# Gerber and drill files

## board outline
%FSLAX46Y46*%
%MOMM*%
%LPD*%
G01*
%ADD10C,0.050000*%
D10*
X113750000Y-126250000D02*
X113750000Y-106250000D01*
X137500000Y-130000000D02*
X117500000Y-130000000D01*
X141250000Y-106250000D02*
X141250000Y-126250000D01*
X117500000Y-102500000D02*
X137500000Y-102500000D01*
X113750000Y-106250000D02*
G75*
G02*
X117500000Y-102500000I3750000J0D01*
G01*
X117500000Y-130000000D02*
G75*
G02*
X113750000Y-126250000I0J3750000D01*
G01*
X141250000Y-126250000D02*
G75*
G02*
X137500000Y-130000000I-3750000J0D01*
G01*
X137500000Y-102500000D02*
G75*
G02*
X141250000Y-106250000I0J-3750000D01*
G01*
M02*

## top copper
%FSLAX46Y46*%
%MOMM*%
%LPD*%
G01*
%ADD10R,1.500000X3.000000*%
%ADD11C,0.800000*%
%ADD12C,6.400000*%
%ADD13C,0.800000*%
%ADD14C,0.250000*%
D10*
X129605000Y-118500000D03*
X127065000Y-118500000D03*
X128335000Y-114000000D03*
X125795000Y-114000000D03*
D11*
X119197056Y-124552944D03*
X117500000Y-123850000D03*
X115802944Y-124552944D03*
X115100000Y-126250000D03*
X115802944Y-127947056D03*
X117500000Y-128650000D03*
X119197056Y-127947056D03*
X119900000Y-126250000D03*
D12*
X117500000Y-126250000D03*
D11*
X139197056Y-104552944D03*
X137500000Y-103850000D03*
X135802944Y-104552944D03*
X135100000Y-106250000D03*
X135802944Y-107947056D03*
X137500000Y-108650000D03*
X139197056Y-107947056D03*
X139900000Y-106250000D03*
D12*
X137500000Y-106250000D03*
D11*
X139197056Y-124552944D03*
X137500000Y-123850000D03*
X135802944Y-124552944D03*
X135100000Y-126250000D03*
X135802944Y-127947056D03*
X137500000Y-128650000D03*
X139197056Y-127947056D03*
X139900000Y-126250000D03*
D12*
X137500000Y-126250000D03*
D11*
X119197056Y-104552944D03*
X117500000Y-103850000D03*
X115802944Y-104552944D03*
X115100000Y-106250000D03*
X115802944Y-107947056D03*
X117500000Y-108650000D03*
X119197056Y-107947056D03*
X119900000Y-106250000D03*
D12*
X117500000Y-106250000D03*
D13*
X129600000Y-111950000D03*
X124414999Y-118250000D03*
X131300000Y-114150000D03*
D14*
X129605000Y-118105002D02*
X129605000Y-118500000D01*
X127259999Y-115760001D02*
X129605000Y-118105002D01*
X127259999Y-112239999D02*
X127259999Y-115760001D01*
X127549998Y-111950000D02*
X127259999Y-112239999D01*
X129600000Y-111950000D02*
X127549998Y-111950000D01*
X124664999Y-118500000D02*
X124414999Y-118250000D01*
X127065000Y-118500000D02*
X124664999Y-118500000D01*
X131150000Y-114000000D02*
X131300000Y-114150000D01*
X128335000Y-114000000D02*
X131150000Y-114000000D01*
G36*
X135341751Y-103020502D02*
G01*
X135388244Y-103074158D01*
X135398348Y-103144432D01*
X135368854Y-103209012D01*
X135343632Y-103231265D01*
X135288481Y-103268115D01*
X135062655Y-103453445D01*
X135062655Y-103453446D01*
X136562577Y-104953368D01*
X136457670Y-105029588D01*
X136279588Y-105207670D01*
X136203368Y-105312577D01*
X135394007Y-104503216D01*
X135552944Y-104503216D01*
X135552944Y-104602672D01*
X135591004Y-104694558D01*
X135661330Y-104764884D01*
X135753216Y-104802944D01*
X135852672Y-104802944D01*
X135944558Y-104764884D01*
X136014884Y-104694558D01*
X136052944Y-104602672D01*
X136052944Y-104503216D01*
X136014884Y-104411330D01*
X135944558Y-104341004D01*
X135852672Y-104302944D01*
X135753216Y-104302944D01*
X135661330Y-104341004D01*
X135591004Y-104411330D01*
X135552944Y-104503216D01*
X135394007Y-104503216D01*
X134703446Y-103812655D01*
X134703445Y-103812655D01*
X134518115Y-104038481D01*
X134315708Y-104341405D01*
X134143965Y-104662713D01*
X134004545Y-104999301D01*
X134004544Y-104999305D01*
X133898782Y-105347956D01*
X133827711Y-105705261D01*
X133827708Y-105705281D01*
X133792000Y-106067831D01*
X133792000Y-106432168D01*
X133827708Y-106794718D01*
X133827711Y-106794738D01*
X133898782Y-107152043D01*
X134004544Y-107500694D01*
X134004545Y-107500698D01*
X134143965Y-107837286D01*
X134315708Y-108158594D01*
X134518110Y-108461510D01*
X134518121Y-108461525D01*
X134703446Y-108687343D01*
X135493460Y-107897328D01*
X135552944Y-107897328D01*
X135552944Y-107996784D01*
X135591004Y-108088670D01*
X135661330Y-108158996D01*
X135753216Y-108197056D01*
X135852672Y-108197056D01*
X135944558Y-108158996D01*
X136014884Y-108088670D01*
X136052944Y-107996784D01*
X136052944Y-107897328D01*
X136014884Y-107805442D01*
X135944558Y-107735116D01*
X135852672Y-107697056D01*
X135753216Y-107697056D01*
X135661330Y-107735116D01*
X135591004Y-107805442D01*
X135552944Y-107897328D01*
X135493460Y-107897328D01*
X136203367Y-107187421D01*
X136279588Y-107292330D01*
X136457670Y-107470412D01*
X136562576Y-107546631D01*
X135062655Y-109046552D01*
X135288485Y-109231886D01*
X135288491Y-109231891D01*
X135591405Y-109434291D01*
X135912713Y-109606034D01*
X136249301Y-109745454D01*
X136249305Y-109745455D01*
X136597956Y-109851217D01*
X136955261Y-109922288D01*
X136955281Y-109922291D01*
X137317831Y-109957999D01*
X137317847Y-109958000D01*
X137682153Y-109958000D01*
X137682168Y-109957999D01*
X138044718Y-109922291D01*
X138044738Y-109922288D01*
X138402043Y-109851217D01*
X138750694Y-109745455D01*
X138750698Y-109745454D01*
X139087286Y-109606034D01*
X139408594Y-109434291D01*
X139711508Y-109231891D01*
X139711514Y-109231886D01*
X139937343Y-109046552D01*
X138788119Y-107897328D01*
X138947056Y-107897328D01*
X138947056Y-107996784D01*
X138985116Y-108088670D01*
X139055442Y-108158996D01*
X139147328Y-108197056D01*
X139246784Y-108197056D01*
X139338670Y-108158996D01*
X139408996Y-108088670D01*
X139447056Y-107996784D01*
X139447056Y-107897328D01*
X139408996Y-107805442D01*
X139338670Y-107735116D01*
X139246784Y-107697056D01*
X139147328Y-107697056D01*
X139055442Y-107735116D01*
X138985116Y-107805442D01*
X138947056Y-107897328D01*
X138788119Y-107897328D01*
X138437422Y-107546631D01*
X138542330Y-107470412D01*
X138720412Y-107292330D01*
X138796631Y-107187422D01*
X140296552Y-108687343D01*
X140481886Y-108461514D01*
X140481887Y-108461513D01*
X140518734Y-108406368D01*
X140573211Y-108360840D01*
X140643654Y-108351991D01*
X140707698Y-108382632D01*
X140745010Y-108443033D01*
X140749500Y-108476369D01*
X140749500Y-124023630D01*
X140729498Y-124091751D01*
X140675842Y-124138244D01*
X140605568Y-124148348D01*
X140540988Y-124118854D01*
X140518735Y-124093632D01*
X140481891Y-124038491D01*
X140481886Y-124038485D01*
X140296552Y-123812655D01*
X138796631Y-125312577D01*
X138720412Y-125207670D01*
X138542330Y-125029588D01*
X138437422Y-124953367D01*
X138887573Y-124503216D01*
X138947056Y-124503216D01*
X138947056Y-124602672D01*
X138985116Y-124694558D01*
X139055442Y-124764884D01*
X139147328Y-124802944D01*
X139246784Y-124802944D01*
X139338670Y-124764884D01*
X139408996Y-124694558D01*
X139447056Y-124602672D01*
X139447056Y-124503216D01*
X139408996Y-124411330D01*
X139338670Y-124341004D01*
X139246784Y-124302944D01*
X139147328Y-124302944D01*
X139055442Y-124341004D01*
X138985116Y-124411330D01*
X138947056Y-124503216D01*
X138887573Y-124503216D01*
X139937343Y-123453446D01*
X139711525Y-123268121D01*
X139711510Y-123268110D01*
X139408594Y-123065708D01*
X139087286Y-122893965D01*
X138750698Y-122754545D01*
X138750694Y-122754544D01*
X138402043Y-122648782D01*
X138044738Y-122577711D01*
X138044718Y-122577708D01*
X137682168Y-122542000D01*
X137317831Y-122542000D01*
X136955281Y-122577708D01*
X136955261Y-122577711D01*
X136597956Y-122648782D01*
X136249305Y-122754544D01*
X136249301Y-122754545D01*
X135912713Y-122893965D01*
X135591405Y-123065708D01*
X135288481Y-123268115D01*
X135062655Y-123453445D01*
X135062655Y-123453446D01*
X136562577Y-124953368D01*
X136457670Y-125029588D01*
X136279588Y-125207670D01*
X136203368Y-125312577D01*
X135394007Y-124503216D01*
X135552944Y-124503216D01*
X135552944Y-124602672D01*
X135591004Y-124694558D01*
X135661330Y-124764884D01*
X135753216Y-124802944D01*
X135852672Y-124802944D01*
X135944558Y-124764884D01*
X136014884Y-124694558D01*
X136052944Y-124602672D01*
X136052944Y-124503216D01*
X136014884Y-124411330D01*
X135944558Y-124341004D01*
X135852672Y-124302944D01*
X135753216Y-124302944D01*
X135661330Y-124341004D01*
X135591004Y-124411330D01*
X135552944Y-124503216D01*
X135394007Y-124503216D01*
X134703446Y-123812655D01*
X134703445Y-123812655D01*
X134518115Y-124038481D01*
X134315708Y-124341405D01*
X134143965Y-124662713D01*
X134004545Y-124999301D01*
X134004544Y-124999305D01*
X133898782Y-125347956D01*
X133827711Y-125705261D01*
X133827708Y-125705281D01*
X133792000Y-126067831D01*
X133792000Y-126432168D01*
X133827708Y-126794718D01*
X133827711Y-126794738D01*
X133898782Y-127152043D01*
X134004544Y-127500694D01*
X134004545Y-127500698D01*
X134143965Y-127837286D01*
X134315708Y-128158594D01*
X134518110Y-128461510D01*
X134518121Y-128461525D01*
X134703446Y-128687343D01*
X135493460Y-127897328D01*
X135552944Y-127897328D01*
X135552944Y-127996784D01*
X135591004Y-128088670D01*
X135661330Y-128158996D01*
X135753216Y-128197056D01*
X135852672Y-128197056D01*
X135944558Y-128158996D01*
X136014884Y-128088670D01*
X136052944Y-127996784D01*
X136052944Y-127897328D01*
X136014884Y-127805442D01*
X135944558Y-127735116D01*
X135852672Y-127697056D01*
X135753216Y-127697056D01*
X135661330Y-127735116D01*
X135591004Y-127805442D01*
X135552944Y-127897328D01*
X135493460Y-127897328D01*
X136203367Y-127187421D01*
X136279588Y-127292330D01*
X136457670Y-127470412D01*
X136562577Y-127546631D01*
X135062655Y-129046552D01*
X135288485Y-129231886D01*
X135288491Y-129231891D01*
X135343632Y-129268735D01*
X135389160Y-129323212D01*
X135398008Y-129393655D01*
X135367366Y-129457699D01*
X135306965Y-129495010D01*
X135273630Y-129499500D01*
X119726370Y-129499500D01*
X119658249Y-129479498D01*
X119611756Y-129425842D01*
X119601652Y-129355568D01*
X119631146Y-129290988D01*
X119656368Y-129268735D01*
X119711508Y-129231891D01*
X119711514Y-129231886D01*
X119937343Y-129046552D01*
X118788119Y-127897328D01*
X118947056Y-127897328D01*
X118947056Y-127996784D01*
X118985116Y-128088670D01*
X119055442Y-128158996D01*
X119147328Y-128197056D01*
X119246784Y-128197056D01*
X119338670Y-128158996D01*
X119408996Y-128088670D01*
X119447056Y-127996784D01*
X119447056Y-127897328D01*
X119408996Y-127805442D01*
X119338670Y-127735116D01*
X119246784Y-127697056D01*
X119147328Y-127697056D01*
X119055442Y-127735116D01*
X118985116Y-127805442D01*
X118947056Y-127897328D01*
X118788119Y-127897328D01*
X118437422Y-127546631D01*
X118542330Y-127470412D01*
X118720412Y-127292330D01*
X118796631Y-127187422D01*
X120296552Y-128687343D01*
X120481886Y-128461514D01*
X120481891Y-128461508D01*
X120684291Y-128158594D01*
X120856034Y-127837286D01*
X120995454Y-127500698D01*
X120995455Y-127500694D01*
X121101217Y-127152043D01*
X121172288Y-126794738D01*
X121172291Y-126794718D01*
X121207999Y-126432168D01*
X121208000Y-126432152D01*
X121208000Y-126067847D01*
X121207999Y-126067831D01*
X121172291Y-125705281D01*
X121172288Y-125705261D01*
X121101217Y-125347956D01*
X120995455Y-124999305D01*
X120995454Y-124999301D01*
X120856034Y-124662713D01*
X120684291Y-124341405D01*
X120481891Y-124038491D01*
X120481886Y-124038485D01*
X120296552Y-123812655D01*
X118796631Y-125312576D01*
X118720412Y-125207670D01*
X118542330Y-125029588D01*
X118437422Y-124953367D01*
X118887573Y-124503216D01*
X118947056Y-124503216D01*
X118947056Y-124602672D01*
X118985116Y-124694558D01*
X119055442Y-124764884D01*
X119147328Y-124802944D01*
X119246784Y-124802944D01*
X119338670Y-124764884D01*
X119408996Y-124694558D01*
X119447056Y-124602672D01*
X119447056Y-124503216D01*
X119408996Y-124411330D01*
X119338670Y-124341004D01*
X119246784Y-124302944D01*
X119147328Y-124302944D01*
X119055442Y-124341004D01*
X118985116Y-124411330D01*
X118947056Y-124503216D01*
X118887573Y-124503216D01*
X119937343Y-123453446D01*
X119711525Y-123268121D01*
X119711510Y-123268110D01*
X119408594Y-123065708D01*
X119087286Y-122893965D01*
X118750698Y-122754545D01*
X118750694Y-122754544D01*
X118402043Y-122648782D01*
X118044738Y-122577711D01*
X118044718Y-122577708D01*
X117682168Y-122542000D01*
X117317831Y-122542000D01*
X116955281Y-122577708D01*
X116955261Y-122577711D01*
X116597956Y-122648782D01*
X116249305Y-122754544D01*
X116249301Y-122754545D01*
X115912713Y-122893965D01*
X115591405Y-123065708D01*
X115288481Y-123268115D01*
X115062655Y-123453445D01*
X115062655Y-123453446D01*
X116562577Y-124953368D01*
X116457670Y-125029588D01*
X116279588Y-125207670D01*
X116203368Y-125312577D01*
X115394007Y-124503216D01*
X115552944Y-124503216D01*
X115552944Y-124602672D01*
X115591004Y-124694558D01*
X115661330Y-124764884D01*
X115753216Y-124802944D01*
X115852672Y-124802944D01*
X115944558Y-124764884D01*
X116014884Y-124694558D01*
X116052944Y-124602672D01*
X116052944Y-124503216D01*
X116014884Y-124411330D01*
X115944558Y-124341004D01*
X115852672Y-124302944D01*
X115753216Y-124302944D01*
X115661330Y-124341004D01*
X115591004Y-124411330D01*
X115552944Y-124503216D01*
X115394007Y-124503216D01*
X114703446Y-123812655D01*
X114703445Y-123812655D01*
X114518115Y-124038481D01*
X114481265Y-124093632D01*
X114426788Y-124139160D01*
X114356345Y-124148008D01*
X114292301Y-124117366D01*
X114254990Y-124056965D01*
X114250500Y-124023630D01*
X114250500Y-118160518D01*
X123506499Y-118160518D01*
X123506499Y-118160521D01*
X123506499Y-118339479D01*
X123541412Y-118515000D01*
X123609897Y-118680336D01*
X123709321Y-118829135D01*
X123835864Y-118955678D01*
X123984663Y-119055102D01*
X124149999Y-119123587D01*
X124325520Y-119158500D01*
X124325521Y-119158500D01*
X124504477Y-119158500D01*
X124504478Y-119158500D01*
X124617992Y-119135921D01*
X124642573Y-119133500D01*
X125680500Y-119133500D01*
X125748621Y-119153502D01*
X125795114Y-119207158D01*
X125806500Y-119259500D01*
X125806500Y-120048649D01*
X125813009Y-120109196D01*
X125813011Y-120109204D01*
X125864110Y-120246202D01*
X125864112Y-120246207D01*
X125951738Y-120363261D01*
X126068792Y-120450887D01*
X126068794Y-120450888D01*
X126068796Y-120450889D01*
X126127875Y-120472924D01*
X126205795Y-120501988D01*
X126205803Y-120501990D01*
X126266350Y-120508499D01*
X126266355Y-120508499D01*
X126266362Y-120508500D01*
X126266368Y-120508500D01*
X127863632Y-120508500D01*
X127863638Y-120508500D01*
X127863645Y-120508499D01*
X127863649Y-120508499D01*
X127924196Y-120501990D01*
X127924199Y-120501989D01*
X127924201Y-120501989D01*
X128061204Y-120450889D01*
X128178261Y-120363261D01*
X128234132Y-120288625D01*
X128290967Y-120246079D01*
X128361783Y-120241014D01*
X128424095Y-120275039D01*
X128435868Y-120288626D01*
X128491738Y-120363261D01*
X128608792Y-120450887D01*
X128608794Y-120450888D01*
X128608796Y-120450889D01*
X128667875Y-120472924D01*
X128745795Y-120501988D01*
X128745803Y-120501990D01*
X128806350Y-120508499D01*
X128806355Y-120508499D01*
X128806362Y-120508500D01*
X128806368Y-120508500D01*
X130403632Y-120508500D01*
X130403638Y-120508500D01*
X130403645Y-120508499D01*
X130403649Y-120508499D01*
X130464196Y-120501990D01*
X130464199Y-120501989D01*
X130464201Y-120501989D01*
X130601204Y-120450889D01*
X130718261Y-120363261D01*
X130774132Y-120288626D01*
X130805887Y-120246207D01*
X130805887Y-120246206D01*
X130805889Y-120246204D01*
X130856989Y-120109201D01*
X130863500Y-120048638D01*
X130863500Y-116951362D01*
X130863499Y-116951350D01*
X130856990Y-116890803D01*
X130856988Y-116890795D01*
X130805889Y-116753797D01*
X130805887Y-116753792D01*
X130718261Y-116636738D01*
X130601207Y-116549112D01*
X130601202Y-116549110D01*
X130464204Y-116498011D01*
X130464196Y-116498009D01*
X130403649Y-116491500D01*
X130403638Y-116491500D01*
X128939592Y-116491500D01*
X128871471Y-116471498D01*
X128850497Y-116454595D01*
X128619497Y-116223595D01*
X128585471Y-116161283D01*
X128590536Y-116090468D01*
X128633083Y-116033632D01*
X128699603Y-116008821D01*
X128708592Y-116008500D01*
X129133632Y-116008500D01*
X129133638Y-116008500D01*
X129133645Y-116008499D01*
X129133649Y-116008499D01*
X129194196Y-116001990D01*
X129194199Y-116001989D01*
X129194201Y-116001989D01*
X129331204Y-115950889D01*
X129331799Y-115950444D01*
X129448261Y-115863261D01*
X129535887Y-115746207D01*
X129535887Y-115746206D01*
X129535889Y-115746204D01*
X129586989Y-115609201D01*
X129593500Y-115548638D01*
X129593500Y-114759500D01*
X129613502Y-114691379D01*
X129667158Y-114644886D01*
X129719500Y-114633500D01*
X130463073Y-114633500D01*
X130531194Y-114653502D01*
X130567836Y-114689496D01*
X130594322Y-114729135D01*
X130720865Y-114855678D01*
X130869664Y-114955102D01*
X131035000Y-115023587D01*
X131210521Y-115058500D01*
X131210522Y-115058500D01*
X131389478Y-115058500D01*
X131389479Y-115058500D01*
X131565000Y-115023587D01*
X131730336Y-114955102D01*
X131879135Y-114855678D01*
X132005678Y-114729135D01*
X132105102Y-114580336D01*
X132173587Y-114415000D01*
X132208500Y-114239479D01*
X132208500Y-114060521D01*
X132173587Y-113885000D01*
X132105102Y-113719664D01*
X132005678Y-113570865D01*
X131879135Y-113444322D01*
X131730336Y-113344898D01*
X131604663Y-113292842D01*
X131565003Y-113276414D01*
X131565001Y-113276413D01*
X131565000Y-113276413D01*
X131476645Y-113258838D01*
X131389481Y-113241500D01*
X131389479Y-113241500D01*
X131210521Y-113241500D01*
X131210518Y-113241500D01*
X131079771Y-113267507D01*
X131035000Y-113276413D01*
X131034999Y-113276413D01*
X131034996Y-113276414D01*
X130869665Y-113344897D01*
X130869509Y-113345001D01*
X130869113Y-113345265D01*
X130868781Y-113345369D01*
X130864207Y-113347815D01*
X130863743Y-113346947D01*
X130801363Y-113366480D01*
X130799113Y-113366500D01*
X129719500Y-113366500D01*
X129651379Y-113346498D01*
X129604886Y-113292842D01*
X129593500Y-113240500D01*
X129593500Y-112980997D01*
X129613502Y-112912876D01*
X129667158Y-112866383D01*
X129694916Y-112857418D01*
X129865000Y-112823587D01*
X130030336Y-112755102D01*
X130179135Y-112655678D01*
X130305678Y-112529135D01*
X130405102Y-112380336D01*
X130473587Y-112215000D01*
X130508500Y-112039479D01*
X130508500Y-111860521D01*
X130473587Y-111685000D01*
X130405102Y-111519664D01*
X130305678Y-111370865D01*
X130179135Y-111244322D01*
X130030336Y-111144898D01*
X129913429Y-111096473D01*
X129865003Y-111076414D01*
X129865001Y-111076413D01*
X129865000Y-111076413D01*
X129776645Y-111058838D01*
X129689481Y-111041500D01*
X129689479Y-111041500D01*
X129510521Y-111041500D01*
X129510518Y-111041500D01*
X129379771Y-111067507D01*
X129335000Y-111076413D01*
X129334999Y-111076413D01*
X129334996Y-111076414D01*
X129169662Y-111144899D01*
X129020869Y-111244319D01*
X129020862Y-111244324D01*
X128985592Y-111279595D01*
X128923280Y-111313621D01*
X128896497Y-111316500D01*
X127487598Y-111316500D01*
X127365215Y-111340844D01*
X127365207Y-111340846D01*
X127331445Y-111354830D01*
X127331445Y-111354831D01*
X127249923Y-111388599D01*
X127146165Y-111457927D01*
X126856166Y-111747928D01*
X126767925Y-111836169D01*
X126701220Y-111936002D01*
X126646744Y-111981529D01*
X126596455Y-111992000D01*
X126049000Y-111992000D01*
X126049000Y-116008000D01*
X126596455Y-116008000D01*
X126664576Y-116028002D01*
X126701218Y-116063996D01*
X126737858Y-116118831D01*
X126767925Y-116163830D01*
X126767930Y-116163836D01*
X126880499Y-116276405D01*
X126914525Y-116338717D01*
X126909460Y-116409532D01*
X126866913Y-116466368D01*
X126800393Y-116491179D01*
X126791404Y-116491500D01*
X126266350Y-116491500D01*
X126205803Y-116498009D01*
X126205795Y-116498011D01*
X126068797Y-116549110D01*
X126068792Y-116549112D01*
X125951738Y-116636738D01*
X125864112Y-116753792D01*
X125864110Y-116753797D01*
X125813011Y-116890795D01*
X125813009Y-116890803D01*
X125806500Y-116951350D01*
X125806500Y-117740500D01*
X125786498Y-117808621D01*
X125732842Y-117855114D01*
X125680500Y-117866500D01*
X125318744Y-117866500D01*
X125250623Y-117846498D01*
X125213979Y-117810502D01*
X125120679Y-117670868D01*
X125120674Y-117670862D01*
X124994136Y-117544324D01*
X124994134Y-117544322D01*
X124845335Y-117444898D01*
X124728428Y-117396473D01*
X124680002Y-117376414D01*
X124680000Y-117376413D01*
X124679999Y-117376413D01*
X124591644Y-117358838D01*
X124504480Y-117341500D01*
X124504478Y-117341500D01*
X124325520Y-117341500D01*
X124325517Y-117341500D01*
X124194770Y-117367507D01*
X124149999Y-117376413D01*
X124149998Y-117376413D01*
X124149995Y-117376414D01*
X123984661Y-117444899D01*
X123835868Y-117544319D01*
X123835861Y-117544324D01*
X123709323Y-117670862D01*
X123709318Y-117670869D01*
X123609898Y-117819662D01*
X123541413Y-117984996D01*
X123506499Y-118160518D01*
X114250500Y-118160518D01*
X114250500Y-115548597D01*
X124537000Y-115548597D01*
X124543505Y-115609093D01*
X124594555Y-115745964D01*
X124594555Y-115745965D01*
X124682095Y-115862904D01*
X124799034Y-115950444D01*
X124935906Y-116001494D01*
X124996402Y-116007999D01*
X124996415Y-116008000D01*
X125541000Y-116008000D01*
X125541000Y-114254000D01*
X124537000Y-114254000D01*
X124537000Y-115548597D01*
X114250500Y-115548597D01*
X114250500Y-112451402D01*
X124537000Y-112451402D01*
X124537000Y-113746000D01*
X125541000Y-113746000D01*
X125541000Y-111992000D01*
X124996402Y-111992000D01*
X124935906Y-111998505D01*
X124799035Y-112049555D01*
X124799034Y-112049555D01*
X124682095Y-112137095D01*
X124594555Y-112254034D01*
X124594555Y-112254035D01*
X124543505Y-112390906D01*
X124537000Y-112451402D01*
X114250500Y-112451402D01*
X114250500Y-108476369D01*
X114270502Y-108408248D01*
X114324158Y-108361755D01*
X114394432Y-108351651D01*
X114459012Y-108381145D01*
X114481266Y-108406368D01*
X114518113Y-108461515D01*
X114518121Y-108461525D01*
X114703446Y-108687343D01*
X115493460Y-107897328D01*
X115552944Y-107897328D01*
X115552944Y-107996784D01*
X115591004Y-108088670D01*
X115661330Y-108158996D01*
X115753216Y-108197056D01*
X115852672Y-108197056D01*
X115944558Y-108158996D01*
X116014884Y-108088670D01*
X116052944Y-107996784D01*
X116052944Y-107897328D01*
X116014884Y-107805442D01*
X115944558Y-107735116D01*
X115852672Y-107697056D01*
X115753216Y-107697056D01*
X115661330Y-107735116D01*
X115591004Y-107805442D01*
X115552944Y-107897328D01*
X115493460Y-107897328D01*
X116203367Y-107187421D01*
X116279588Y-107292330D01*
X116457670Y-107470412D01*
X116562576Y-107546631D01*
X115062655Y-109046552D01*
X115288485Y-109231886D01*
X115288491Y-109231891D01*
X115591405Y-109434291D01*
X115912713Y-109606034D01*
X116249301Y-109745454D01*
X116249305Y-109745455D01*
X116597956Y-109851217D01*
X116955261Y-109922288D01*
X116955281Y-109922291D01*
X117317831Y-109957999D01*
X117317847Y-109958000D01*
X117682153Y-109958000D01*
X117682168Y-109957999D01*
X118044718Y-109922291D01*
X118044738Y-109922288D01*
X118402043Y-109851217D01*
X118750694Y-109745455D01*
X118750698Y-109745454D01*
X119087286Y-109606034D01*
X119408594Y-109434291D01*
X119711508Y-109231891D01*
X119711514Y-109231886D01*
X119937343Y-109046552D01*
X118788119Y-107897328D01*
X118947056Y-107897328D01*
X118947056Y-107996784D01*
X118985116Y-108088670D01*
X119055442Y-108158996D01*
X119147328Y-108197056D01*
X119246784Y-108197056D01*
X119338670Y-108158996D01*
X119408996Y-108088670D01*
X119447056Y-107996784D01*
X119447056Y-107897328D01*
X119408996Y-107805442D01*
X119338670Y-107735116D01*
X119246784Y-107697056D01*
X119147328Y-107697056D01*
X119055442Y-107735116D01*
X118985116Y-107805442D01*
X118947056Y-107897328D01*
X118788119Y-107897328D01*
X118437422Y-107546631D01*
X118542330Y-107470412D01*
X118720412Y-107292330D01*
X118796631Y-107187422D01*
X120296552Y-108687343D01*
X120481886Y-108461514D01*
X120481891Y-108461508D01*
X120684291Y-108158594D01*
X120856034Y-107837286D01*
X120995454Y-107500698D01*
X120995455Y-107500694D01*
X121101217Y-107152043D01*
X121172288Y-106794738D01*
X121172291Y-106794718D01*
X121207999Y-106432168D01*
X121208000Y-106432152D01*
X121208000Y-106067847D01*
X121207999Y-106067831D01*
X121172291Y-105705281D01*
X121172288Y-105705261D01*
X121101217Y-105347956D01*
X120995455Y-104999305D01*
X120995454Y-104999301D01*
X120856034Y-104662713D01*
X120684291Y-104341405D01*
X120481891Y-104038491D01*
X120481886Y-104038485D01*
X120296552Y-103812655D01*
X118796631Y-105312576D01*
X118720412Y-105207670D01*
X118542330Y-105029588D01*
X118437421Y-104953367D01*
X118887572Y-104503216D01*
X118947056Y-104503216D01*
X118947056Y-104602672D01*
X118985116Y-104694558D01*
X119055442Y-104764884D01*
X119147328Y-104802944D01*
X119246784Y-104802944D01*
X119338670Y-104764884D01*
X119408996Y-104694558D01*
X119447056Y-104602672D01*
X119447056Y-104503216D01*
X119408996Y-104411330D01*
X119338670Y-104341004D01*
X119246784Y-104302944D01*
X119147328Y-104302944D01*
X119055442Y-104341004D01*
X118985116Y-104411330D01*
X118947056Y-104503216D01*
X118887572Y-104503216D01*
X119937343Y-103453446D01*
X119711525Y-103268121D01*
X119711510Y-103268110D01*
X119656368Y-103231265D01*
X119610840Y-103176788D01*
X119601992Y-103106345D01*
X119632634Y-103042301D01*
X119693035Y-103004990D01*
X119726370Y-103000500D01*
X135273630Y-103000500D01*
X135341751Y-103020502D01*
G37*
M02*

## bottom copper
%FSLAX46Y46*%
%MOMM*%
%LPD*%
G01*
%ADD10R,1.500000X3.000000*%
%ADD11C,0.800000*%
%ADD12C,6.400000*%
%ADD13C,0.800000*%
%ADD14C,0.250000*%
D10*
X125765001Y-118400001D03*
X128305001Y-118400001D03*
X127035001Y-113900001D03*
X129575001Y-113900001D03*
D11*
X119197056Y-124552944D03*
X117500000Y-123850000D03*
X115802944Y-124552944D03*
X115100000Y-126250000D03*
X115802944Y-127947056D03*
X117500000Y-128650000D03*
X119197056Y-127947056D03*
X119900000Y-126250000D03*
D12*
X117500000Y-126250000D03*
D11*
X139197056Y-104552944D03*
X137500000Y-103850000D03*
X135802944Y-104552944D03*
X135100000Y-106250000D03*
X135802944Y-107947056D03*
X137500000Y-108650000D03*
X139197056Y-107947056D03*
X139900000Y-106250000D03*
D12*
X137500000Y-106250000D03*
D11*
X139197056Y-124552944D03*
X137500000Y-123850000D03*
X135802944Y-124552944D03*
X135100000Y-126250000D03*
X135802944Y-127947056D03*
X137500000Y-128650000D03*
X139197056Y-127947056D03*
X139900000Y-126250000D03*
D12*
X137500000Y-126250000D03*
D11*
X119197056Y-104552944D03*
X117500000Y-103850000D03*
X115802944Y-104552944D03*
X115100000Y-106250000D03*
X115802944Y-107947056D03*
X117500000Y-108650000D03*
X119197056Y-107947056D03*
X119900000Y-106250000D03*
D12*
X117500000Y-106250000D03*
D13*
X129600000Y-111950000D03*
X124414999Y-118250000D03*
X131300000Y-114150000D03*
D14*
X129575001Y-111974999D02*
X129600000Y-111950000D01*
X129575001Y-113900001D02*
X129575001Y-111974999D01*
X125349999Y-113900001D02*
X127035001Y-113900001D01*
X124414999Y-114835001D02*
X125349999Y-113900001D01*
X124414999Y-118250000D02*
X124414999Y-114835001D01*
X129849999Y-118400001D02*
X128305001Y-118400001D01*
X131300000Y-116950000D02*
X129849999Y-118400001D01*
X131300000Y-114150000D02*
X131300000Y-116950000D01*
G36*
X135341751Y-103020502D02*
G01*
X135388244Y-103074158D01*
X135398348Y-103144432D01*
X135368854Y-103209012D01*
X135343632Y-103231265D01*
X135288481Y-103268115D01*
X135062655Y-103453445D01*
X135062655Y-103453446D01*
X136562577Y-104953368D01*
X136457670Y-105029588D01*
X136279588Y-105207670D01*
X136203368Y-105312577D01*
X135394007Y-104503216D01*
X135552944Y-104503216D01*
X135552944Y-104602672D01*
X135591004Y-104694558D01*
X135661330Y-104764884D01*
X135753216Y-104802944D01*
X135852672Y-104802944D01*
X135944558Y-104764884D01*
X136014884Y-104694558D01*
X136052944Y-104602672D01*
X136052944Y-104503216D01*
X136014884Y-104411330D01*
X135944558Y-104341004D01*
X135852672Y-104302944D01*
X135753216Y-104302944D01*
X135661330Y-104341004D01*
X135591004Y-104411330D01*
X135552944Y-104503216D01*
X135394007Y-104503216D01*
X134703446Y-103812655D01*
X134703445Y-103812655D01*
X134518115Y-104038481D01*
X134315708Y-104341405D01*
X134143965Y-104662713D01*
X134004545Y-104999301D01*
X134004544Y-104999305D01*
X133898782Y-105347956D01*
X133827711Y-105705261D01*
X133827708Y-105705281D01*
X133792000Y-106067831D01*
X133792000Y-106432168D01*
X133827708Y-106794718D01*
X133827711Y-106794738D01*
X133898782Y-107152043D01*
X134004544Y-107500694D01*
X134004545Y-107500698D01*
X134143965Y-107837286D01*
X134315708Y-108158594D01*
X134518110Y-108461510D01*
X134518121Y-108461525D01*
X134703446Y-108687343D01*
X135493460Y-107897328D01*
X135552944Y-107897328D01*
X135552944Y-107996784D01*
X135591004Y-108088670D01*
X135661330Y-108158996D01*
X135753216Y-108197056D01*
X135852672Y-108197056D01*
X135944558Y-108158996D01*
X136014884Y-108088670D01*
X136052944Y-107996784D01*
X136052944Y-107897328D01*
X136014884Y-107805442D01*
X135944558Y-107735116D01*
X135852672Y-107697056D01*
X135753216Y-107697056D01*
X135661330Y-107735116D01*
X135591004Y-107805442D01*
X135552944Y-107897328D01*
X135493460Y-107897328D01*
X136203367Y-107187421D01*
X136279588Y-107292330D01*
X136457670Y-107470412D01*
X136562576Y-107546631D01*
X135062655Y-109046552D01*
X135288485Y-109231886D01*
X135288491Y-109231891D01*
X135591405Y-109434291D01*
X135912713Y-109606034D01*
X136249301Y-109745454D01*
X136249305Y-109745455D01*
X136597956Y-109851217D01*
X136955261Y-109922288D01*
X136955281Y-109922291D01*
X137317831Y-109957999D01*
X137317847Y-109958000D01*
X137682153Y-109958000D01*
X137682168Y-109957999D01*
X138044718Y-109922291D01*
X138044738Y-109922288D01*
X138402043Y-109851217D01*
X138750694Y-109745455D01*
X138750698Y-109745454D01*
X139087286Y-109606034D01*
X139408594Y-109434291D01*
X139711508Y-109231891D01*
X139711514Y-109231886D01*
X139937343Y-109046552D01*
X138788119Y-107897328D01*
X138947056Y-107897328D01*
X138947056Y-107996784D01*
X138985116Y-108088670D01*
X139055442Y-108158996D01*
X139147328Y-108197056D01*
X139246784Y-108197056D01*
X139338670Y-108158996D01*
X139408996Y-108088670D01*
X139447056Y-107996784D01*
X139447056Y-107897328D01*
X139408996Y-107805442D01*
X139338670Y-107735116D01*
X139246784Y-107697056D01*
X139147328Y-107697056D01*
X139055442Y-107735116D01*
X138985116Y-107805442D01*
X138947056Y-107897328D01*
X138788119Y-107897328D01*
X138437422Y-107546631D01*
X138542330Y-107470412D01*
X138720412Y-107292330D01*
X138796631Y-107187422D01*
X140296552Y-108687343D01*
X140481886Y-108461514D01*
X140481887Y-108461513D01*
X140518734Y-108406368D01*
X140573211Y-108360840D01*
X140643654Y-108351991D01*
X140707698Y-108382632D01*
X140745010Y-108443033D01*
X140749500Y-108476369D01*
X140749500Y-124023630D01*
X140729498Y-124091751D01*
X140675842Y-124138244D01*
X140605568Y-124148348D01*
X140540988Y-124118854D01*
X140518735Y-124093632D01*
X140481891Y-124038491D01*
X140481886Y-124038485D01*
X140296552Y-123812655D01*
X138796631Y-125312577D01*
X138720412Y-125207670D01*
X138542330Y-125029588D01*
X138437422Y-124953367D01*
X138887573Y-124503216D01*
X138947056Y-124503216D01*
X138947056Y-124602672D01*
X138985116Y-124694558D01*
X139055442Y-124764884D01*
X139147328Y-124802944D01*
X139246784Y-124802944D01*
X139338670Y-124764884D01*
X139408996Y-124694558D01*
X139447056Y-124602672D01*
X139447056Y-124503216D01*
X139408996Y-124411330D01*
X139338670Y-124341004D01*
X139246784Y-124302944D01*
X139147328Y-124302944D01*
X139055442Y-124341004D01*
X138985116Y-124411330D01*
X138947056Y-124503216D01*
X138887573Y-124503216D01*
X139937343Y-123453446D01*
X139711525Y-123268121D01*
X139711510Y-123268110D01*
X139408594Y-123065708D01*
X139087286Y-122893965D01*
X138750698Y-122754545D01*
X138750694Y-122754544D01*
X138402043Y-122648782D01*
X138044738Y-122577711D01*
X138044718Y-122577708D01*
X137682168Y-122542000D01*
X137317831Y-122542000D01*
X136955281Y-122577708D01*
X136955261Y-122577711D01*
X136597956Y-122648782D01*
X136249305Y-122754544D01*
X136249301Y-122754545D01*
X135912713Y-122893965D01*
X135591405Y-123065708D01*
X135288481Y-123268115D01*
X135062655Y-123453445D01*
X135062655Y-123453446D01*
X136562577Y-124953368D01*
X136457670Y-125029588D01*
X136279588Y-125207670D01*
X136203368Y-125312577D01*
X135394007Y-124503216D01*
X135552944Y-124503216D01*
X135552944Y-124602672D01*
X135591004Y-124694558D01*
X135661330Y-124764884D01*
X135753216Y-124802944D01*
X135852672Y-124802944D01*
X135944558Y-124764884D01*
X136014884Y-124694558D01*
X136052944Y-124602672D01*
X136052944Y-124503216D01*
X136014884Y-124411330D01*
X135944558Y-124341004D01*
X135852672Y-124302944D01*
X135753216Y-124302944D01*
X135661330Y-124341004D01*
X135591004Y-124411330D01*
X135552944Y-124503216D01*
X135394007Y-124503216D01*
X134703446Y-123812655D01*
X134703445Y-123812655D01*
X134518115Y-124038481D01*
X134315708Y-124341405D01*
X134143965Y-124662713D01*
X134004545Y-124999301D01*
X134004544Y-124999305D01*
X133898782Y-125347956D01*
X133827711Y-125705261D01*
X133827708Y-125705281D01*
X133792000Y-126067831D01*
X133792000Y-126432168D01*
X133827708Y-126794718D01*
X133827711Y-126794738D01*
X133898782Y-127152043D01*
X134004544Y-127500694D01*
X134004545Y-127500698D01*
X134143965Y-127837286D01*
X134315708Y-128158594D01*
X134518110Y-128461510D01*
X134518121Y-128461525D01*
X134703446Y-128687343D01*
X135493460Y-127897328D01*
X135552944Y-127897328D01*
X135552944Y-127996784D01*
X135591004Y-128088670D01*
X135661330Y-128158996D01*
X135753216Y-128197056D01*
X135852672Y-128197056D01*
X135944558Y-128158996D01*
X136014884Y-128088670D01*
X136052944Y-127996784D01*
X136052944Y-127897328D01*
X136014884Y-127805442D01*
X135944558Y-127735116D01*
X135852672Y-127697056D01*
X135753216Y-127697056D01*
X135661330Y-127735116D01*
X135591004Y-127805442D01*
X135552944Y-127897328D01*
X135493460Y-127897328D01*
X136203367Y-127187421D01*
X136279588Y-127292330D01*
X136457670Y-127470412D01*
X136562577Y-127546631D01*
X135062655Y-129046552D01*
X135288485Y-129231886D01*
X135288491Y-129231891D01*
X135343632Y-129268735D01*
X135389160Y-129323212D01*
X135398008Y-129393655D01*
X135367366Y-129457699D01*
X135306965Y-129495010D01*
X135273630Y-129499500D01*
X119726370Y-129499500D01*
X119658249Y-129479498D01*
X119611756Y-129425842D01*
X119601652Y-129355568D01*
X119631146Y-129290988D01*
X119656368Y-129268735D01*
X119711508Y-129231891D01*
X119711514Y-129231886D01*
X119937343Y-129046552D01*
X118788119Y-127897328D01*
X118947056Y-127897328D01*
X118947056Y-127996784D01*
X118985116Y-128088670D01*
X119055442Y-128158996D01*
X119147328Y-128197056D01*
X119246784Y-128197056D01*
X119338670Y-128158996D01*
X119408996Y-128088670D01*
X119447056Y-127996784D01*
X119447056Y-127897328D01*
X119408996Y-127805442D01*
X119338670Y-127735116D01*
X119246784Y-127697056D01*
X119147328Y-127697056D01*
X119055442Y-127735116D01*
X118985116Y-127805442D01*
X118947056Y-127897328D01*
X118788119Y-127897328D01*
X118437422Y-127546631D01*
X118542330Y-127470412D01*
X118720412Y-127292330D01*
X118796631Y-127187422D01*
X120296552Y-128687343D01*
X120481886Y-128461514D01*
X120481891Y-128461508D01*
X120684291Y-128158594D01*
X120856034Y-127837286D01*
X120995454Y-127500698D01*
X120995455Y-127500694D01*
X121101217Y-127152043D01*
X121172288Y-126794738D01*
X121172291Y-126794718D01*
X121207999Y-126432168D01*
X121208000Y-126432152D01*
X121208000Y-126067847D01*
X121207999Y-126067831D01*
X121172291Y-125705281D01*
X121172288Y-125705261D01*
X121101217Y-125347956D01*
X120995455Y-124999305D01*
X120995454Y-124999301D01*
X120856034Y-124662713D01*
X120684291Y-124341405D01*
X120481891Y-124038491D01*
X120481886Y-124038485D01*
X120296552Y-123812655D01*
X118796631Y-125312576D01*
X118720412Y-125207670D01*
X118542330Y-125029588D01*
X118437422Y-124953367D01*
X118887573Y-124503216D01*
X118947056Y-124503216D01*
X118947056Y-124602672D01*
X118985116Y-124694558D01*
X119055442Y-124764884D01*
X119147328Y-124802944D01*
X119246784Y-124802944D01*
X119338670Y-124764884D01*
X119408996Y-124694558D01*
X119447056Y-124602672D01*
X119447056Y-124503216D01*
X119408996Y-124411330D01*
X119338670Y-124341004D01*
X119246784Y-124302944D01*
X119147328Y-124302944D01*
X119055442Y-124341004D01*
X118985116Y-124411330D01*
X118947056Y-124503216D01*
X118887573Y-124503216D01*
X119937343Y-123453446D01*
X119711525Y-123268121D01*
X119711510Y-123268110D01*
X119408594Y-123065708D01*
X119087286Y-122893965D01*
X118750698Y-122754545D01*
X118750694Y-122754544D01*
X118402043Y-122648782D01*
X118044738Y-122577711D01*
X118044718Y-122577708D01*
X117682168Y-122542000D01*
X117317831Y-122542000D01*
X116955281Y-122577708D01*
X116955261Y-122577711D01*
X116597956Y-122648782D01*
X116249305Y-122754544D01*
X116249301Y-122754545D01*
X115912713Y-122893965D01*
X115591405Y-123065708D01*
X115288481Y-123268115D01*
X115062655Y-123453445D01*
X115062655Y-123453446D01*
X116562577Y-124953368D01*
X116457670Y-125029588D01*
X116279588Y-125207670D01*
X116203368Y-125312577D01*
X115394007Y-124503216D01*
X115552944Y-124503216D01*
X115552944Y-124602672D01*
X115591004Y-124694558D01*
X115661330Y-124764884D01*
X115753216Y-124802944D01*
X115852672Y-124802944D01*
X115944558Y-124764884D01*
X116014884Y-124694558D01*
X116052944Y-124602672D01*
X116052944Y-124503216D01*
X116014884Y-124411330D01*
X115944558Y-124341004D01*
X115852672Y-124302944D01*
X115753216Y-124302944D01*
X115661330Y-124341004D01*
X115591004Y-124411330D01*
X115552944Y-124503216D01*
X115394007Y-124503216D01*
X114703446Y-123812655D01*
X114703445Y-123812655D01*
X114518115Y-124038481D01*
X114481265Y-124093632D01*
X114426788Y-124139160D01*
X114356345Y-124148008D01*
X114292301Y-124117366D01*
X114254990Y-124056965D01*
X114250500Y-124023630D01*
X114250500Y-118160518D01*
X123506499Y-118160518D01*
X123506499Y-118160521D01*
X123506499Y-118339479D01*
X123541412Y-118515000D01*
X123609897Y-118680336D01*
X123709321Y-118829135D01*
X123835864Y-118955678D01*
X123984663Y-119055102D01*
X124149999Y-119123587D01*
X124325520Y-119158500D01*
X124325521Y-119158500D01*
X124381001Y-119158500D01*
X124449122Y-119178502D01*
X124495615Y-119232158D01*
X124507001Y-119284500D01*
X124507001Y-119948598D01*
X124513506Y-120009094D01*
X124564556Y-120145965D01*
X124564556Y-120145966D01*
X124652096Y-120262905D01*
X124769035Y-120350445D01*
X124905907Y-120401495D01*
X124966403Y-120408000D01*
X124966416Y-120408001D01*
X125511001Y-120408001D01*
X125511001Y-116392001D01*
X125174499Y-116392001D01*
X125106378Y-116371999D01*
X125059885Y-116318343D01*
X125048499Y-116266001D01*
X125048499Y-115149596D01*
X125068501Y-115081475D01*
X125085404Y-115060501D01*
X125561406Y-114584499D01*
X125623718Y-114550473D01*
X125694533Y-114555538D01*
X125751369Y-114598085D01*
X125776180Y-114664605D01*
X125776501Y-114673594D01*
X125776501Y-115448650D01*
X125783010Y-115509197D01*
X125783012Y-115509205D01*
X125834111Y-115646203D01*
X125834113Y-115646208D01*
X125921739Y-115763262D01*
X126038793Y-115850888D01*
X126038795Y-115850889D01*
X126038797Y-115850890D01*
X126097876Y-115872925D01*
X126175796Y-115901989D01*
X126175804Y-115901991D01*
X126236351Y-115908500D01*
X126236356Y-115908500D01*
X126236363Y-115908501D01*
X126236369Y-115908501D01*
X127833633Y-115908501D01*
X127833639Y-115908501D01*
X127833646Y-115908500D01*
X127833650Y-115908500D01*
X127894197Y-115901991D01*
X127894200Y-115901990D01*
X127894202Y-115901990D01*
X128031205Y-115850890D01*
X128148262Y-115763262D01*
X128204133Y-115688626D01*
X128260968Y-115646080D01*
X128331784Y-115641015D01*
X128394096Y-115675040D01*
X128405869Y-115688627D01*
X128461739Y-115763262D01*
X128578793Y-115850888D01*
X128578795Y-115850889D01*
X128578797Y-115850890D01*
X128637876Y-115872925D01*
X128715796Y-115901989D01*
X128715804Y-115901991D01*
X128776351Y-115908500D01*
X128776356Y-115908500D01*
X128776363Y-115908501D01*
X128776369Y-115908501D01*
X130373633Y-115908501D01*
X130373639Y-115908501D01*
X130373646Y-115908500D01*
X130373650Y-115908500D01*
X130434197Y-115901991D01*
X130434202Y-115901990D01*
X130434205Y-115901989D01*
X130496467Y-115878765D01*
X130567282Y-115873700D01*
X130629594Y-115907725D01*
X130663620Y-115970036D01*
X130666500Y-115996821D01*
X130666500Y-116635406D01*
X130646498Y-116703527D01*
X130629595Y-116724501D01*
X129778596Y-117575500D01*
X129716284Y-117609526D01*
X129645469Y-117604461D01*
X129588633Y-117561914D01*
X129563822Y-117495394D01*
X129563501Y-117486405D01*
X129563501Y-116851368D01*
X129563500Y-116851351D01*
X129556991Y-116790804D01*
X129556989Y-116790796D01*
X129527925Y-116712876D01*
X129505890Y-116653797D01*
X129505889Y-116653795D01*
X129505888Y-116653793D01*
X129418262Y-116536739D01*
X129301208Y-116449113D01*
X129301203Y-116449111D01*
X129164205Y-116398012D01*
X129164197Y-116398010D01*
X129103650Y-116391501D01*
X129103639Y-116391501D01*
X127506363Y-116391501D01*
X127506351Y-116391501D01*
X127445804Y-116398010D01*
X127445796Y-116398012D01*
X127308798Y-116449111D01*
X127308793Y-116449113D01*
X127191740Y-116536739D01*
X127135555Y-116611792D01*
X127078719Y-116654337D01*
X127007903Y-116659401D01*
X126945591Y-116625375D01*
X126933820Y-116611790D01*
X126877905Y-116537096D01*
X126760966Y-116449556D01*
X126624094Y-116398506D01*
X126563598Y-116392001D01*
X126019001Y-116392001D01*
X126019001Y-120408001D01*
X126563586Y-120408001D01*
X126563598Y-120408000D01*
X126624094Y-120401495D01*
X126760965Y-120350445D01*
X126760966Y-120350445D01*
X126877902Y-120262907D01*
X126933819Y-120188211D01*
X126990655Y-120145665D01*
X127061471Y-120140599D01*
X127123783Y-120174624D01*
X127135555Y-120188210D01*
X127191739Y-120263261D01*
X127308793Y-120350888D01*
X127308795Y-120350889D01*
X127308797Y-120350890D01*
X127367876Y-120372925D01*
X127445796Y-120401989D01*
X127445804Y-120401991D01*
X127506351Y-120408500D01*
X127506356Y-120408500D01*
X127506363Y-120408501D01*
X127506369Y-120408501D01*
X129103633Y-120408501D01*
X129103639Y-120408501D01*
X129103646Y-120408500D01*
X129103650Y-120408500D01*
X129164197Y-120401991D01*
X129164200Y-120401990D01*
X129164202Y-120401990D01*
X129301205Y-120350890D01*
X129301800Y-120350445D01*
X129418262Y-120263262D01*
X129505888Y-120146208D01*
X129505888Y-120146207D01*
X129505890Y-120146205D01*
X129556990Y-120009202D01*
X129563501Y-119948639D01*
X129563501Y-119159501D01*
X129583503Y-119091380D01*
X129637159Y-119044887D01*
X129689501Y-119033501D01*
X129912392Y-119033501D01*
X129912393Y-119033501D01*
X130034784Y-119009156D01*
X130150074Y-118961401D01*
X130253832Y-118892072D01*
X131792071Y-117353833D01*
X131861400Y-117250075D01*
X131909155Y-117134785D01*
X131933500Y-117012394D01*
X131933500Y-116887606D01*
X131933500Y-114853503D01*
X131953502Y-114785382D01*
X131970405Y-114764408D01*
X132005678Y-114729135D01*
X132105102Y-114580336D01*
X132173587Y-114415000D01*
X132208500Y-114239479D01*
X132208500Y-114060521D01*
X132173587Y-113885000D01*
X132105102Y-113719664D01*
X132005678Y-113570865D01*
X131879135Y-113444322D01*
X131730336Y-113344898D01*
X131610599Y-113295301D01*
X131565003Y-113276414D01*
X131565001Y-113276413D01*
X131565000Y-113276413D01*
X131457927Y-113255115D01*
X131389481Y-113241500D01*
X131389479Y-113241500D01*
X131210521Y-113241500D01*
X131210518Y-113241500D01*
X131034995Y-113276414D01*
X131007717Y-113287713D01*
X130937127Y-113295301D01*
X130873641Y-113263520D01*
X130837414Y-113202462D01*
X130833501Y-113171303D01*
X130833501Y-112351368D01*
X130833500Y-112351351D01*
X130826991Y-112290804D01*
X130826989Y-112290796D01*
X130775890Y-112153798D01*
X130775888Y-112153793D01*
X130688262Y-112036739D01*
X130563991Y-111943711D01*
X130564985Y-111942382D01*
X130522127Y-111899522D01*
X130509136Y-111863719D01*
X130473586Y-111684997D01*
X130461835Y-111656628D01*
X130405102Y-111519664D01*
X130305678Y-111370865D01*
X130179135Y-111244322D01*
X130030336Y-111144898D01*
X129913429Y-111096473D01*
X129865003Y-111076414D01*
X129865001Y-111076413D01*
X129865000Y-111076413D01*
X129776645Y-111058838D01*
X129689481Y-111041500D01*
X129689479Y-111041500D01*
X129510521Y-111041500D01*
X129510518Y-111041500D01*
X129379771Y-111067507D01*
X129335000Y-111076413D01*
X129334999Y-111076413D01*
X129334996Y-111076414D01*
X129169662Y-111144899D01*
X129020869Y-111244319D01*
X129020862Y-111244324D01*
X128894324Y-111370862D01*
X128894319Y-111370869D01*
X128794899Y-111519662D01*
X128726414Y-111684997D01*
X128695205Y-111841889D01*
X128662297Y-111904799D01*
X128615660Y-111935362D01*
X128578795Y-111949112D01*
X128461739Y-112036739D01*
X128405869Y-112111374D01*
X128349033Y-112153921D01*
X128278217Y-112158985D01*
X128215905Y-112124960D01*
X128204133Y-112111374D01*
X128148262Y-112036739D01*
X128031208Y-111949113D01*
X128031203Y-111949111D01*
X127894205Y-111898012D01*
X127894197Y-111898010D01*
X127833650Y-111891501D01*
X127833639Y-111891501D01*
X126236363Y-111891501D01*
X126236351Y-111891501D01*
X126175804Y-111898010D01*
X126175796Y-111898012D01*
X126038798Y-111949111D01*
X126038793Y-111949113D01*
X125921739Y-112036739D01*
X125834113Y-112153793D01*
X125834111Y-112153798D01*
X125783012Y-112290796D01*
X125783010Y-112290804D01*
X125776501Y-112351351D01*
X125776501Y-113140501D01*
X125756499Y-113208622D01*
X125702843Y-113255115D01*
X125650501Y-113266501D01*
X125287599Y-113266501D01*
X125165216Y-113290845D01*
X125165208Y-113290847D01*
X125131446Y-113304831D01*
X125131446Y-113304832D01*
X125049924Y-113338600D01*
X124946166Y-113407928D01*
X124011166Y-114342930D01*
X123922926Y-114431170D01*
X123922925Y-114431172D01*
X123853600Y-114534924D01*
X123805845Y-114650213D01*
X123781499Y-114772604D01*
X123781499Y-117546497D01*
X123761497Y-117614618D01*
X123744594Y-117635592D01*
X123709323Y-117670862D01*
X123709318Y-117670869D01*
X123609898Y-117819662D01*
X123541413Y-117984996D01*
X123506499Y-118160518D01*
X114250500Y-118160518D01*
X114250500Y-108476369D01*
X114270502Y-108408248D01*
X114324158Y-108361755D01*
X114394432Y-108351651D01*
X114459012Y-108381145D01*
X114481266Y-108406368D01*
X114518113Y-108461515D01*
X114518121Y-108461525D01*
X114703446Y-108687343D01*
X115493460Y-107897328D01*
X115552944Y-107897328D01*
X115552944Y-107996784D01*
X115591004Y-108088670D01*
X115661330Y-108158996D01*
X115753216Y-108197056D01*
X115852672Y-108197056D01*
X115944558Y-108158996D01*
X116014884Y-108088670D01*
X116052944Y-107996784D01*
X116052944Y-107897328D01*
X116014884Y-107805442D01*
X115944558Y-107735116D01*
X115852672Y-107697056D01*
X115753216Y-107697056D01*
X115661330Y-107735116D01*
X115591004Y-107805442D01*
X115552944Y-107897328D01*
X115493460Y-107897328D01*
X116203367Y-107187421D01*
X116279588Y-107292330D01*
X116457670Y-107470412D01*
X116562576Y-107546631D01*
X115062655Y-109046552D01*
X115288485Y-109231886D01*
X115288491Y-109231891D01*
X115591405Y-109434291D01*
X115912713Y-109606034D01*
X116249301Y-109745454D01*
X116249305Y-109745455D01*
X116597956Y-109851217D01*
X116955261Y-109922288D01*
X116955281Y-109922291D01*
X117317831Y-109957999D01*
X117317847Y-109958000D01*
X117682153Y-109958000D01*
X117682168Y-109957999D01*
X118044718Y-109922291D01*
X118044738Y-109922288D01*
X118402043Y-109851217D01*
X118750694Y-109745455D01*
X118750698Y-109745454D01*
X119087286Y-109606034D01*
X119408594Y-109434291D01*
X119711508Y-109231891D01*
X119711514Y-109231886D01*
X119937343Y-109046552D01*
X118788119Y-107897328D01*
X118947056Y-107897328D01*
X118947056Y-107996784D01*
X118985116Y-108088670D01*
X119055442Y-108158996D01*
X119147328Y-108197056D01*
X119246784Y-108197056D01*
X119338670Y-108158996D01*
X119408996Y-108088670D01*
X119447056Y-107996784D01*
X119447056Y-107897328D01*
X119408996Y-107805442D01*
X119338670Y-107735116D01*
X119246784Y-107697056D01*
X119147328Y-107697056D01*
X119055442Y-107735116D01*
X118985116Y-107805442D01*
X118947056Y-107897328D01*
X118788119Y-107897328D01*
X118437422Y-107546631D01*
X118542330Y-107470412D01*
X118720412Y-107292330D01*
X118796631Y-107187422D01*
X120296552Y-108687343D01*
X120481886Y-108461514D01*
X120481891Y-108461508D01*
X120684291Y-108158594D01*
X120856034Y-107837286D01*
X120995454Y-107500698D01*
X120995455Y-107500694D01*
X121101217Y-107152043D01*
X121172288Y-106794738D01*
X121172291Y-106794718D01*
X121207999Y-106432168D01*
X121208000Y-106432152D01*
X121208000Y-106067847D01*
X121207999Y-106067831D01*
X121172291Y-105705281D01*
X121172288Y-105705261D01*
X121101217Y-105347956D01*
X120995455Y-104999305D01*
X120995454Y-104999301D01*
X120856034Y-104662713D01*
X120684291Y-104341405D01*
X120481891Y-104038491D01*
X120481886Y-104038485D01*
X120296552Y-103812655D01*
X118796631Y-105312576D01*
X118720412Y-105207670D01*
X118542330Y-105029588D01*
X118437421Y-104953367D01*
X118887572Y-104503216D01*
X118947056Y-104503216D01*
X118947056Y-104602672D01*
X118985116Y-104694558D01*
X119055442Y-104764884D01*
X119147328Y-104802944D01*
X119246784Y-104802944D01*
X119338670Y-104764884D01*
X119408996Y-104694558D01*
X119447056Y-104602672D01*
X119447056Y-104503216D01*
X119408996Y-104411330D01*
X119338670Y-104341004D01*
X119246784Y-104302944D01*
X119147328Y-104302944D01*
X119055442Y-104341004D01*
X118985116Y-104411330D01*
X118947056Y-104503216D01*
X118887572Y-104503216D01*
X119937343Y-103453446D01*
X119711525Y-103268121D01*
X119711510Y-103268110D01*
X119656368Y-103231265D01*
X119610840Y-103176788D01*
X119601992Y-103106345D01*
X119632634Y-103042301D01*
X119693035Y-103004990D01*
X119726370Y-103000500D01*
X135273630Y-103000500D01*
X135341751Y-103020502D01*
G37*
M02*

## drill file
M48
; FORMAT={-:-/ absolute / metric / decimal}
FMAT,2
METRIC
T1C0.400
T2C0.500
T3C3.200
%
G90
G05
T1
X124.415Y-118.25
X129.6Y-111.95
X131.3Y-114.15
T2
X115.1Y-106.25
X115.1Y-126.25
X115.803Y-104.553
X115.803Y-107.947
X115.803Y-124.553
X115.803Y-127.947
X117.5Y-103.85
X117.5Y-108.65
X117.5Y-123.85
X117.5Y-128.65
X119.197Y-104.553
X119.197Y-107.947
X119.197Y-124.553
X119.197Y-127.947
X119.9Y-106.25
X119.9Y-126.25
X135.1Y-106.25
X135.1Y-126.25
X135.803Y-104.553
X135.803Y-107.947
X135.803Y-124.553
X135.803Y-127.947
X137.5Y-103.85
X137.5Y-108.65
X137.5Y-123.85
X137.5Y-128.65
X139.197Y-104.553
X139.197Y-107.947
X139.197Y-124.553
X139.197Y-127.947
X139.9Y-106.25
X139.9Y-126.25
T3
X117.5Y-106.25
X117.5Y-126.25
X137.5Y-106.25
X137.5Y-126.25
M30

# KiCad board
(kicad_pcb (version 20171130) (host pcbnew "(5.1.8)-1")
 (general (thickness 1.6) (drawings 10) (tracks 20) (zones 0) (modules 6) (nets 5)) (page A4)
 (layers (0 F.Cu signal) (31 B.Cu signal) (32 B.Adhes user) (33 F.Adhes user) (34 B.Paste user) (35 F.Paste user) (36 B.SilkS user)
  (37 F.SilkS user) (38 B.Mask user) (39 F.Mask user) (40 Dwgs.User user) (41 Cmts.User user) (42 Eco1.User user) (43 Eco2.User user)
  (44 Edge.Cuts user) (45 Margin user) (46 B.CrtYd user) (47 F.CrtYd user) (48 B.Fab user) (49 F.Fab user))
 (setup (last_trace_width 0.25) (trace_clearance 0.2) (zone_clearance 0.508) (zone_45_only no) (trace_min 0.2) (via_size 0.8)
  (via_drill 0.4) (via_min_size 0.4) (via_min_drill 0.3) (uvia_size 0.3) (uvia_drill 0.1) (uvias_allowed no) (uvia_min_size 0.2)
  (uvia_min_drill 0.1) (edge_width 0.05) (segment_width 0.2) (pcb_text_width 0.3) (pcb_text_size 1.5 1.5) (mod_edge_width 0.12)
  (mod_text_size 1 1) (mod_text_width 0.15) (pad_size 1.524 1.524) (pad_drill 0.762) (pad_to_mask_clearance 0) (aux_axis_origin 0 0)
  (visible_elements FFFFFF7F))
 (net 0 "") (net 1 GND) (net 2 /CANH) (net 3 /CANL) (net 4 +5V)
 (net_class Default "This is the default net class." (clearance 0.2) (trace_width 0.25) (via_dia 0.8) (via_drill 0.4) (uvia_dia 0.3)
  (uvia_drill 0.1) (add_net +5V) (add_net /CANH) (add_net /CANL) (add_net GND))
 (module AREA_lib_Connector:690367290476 (layer B.Cu) (at 127.670001 116.150001)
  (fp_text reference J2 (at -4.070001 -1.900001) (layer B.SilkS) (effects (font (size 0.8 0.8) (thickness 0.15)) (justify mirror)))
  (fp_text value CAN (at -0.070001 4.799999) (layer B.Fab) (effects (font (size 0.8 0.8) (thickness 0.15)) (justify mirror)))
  (pad 4 smd rect (at -1.905 2.25) (size 1.5 3) (layers B.Cu B.Paste B.Mask) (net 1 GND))
  (pad 2 smd rect (at 0.635 2.25) (size 1.5 3) (layers B.Cu B.Paste B.Mask) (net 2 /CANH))
  (pad 3 smd rect (at -0.635 -2.25) (size 1.5 3) (layers B.Cu B.Paste B.Mask) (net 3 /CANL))
  (pad 1 smd rect (at 1.905 -2.25) (size 1.5 3) (layers B.Cu B.Paste B.Mask) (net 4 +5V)))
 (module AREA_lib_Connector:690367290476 (layer F.Cu) (at 127.7 116.25)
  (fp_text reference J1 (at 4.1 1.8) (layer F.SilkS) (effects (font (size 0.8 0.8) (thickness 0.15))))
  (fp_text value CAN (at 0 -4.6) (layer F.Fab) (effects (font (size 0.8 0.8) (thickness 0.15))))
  (pad 1 smd rect (at 1.905 2.25) (size 1.5 3) (layers F.Cu F.Paste F.Mask) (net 4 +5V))
  (pad 3 smd rect (at -0.635 2.25) (size 1.5 3) (layers F.Cu F.Paste F.Mask) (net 3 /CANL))
  (pad 2 smd rect (at 0.635 -2.25) (size 1.5 3) (layers F.Cu F.Paste F.Mask) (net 2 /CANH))
  (pad 4 smd rect (at -1.905 -2.25) (size 1.5 3) (layers F.Cu F.Paste F.Mask) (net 1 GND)))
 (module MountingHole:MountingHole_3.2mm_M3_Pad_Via (layer F.Cu) (at 117.5 126.25)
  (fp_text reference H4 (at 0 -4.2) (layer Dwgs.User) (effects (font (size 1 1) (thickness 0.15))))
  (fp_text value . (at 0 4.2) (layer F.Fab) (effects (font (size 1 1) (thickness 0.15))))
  (pad 1 thru_hole circle (at 1.697056 -1.697056) (size 0.8 0.8) (drill 0.5) (layers *.Cu *.Mask) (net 1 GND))
  (pad 1 thru_hole circle (at 0 -2.4) (size 0.8 0.8) (drill 0.5) (layers *.Cu *.Mask) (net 1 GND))
  (pad 1 thru_hole circle (at -1.697056 -1.697056) (size 0.8 0.8) (drill 0.5) (layers *.Cu *.Mask) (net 1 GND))
  (pad 1 thru_hole circle (at -2.4 0) (size 0.8 0.8) (drill 0.5) (layers *.Cu *.Mask) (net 1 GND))
  (pad 1 thru_hole circle (at -1.697056 1.697056) (size 0.8 0.8) (drill 0.5) (layers *.Cu *.Mask) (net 1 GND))
  (pad 1 thru_hole circle (at 0 2.4) (size 0.8 0.8) (drill 0.5) (layers *.Cu *.Mask) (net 1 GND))
  (pad 1 thru_hole circle (at 1.697056 1.697056) (size 0.8 0.8) (drill 0.5) (layers *.Cu *.Mask) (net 1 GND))
  (pad 1 thru_hole circle (at 2.4 0) (size 0.8 0.8) (drill 0.5) (layers *.Cu *.Mask) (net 1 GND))
  (pad 1 thru_hole circle (at 0 0) (size 6.4 6.4) (drill 3.2) (layers *.Cu *.Mask) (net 1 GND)))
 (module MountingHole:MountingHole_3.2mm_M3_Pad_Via (layer F.Cu) (at 137.5 106.25)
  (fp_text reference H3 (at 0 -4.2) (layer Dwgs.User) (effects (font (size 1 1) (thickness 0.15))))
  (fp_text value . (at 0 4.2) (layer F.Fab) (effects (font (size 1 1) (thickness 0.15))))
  (pad 1 thru_hole circle (at 1.697056 -1.697056) (size 0.8 0.8) (drill 0.5) (layers *.Cu *.Mask) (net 1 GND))
  (pad 1 thru_hole circle (at 0 -2.4) (size 0.8 0.8) (drill 0.5) (layers *.Cu *.Mask) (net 1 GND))
  (pad 1 thru_hole circle (at -1.697056 -1.697056) (size 0.8 0.8) (drill 0.5) (layers *.Cu *.Mask) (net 1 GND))
  (pad 1 thru_hole circle (at -2.4 0) (size 0.8 0.8) (drill 0.5) (layers *.Cu *.Mask) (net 1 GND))
  (pad 1 thru_hole circle (at -1.697056 1.697056) (size 0.8 0.8) (drill 0.5) (layers *.Cu *.Mask) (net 1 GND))
  (pad 1 thru_hole circle (at 0 2.4) (size 0.8 0.8) (drill 0.5) (layers *.Cu *.Mask) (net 1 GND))
  (pad 1 thru_hole circle (at 1.697056 1.697056) (size 0.8 0.8) (drill 0.5) (layers *.Cu *.Mask) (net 1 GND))
  (pad 1 thru_hole circle (at 2.4 0) (size 0.8 0.8) (drill 0.5) (layers *.Cu *.Mask) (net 1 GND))
  (pad 1 thru_hole circle (at 0 0) (size 6.4 6.4) (drill 3.2) (layers *.Cu *.Mask) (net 1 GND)))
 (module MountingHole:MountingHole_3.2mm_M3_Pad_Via (layer F.Cu) (at 137.5 126.25)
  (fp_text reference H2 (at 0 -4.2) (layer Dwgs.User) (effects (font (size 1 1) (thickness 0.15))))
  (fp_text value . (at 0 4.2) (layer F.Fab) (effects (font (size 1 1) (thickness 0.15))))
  (pad 1 thru_hole circle (at 1.697056 -1.697056) (size 0.8 0.8) (drill 0.5) (layers *.Cu *.Mask) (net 1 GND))
  (pad 1 thru_hole circle (at 0 -2.4) (size 0.8 0.8) (drill 0.5) (layers *.Cu *.Mask) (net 1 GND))
  (pad 1 thru_hole circle (at -1.697056 -1.697056) (size 0.8 0.8) (drill 0.5) (layers *.Cu *.Mask) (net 1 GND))
  (pad 1 thru_hole circle (at -2.4 0) (size 0.8 0.8) (drill 0.5) (layers *.Cu *.Mask) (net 1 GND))
  (pad 1 thru_hole circle (at -1.697056 1.697056) (size 0.8 0.8) (drill 0.5) (layers *.Cu *.Mask) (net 1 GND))
  (pad 1 thru_hole circle (at 0 2.4) (size 0.8 0.8) (drill 0.5) (layers *.Cu *.Mask) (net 1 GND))
  (pad 1 thru_hole circle (at 1.697056 1.697056) (size 0.8 0.8) (drill 0.5) (layers *.Cu *.Mask) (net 1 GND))
  (pad 1 thru_hole circle (at 2.4 0) (size 0.8 0.8) (drill 0.5) (layers *.Cu *.Mask) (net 1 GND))
  (pad 1 thru_hole circle (at 0 0) (size 6.4 6.4) (drill 3.2) (layers *.Cu *.Mask) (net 1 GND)))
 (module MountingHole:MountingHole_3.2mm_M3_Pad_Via (layer F.Cu) (at 117.5 106.25)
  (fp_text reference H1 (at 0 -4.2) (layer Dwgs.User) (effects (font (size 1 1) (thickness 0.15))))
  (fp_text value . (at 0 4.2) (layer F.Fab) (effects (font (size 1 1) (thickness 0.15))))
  (pad 1 thru_hole circle (at 1.697056 -1.697056) (size 0.8 0.8) (drill 0.5) (layers *.Cu *.Mask) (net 1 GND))
  (pad 1 thru_hole circle (at 0 -2.4) (size 0.8 0.8) (drill 0.5) (layers *.Cu *.Mask) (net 1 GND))
  (pad 1 thru_hole circle (at -1.697056 -1.697056) (size 0.8 0.8) (drill 0.5) (layers *.Cu *.Mask) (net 1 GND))
  (pad 1 thru_hole circle (at -2.4 0) (size 0.8 0.8) (drill 0.5) (layers *.Cu *.Mask) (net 1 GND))
  (pad 1 thru_hole circle (at -1.697056 1.697056) (size 0.8 0.8) (drill 0.5) (layers *.Cu *.Mask) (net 1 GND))
  (pad 1 thru_hole circle (at 0 2.4) (size 0.8 0.8) (drill 0.5) (layers *.Cu *.Mask) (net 1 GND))
  (pad 1 thru_hole circle (at 1.697056 1.697056) (size 0.8 0.8) (drill 0.5) (layers *.Cu *.Mask) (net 1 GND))
  (pad 1 thru_hole circle (at 2.4 0) (size 0.8 0.8) (drill 0.5) (layers *.Cu *.Mask) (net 1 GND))
  (pad 1 thru_hole circle (at 0 0) (size 6.4 6.4) (drill 3.2) (layers *.Cu *.Mask) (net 1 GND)))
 (gr_line (start 113.75 126.25) (end 113.75 106.25) (layer Edge.Cuts) (width 0.05))
 (gr_line (start 137.5 130) (end 117.5 130) (layer Edge.Cuts) (width 0.05))
 (gr_line (start 141.25 106.25) (end 141.25 126.25) (layer Edge.Cuts) (width 0.05))
 (gr_line (start 117.5 102.5) (end 137.5 102.5) (layer Edge.Cuts) (width 0.05))
 (gr_arc (start 117.5 106.25) (end 117.5 102.5) (angle -90) (layer Edge.Cuts) (width 0.05))
 (gr_arc (start 117.5 126.25) (end 113.75 126.25) (angle -90) (layer Edge.Cuts) (width 0.05))
 (gr_arc (start 137.5 126.25) (end 137.5 130) (angle -90) (layer Edge.Cuts) (width 0.05))
 (gr_arc (start 137.5 106.25) (end 141.25 106.25) (angle -90) (layer Edge.Cuts) (width 0.05))
 (via (at 129.6 111.95) (size 0.8) (drill 0.4) (layers F.Cu B.Cu) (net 4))
 (segment (start 129.575001 111.974999) (end 129.6 111.95) (width 0.25) (layer B.Cu) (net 4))
 (segment (start 129.575001 113.900001) (end 129.575001 111.974999) (width 0.25) (layer B.Cu) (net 4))
 (segment (start 129.605 118.105002) (end 129.605 118.5) (width 0.25) (layer F.Cu) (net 4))
 (segment (start 127.259999 115.760001) (end 129.605 118.105002) (width 0.25) (layer F.Cu) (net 4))
 (segment (start 127.259999 112.239999) (end 127.259999 115.760001) (width 0.25) (layer F.Cu) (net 4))
 (segment (start 127.549998 111.95) (end 127.259999 112.239999) (width 0.25) (layer F.Cu) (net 4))
 (segment (start 129.6 111.95) (end 127.549998 111.95) (width 0.25) (layer F.Cu) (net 4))
 (via (at 124.414999 118.25) (size 0.8) (drill 0.4) (layers F.Cu B.Cu) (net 3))
 (segment (start 124.664999 118.5) (end 124.414999 118.25) (width 0.25) (layer F.Cu) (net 3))
 (segment (start 127.065 118.5) (end 124.664999 118.5) (width 0.25) (layer F.Cu) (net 3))
 (segment (start 125.349999 113.900001) (end 127.035001 113.900001) (width 0.25) (layer B.Cu) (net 3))
 (segment (start 124.414999 114.835001) (end 125.349999 113.900001) (width 0.25) (layer B.Cu) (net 3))
 (segment (start 124.414999 118.25) (end 124.414999 114.835001) (width 0.25) (layer B.Cu) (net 3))
 (via (at 131.3 114.15) (size 0.8) (drill 0.4) (layers F.Cu B.Cu) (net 2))
 (segment (start 131.15 114) (end 131.3 114.15) (width 0.25) (layer F.Cu) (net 2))
 (segment (start 128.335 114) (end 131.15 114) (width 0.25) (layer F.Cu) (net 2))
 (segment (start 129.849999 118.400001) (end 128.305001 118.400001) (width 0.25) (layer B.Cu) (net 2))
 (segment (start 131.3 116.95) (end 129.849999 118.400001) (width 0.25) (layer B.Cu) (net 2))
 (segment (start 131.3 114.15) (end 131.3 116.95) (width 0.25) (layer B.Cu) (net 2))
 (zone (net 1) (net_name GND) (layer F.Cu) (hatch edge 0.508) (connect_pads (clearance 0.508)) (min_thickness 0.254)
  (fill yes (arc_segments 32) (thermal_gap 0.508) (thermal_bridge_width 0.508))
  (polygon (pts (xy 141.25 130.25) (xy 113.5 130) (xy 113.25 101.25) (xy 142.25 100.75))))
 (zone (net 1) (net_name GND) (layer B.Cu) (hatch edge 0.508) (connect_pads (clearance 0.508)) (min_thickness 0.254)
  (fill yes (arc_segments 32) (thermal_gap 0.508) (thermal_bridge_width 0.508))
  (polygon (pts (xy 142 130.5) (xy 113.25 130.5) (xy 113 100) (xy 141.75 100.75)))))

